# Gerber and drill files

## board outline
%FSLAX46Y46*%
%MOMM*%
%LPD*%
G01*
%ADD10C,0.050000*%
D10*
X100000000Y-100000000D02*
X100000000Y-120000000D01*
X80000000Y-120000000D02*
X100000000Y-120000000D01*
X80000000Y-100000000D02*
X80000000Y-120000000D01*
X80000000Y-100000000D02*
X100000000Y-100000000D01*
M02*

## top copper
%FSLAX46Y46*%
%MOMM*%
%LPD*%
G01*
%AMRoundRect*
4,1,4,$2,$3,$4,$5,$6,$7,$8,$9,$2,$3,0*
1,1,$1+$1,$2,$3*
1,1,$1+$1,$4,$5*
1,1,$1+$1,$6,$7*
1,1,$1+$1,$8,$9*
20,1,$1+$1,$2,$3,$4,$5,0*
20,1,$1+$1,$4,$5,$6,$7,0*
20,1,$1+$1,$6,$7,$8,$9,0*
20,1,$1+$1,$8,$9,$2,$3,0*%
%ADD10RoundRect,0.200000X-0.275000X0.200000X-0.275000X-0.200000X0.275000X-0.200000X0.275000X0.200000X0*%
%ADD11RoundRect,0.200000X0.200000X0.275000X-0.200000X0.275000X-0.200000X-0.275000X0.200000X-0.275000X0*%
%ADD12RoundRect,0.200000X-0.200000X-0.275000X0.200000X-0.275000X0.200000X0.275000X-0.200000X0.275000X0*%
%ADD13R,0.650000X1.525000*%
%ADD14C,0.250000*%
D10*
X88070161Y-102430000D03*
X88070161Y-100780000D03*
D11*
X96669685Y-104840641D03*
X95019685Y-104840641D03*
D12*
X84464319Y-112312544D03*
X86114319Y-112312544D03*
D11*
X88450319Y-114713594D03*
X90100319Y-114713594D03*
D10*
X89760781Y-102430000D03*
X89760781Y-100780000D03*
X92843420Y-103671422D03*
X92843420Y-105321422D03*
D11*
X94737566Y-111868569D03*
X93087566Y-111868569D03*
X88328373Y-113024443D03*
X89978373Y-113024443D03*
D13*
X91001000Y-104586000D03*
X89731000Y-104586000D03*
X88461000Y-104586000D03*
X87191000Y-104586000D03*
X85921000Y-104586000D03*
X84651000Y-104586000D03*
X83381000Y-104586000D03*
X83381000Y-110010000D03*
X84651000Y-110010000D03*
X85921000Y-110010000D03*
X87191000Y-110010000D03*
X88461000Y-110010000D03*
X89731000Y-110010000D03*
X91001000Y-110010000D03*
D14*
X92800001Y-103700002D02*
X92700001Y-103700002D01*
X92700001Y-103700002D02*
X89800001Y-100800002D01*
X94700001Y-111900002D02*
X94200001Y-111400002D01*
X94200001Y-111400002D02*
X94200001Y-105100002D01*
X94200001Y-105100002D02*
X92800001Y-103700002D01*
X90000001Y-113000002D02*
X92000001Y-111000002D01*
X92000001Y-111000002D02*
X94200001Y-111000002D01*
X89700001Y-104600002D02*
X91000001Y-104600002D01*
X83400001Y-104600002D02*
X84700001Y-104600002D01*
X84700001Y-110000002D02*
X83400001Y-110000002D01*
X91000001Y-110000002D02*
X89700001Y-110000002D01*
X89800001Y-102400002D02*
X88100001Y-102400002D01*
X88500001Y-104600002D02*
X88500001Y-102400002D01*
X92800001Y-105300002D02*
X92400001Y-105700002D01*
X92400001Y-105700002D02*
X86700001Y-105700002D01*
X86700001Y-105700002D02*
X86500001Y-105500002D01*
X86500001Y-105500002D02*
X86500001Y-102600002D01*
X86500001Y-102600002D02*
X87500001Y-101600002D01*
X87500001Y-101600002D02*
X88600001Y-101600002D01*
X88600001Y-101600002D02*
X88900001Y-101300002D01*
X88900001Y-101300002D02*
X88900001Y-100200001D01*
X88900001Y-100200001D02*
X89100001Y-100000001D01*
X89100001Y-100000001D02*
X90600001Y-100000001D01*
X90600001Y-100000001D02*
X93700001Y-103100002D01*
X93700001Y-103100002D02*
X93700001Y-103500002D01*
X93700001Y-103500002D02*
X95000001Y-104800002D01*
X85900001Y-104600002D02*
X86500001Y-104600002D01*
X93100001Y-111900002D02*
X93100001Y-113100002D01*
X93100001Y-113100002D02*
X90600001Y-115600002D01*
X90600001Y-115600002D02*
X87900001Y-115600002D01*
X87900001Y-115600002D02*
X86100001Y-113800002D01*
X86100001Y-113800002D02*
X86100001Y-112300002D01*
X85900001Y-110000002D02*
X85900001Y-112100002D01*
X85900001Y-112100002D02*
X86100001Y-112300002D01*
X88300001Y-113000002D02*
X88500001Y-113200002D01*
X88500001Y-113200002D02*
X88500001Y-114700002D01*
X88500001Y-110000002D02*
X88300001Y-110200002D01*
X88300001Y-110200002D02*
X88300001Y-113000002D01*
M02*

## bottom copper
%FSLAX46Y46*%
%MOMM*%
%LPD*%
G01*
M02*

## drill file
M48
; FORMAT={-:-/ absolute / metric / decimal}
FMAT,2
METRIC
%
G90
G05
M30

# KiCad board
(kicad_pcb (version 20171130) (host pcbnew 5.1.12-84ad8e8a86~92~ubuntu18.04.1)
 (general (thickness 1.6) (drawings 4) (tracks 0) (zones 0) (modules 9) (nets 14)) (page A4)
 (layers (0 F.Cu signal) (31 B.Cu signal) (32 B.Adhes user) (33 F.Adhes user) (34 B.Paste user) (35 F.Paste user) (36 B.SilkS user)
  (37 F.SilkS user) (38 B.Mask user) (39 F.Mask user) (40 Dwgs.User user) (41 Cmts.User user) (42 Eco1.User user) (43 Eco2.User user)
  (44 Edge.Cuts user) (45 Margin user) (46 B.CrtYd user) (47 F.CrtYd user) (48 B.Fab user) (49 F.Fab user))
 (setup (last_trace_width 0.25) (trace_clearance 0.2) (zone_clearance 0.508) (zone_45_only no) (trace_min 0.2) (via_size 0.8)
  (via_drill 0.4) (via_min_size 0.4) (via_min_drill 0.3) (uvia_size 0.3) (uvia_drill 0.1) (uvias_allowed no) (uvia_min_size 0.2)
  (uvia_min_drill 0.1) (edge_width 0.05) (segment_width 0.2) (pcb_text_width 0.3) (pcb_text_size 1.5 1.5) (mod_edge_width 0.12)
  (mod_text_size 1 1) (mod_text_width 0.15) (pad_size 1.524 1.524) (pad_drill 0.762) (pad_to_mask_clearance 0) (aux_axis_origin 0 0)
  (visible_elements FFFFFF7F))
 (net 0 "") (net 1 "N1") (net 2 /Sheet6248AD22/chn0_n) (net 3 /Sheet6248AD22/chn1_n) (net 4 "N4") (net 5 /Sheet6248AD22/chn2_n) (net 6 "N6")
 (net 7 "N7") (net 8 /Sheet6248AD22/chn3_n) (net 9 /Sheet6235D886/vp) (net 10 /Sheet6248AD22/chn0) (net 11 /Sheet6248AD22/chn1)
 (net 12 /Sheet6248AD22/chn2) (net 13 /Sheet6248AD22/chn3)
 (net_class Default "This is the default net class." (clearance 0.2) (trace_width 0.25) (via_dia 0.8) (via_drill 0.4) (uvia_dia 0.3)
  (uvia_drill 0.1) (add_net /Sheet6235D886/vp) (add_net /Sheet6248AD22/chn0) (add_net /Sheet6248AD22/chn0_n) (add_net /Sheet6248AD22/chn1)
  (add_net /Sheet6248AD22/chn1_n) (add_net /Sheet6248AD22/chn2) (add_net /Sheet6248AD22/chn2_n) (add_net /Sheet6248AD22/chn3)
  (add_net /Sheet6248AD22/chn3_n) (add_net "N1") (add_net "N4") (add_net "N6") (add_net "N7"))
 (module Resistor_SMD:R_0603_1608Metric (layer F.Cu) (at 88.070161 101.605000 270.000000)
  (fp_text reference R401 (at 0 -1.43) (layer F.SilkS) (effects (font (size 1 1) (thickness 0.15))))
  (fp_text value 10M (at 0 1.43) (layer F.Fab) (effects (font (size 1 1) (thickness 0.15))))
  (pad 2 smd roundrect (at 0.825 0 270.000000) (size 0.8 0.95) (layers F.Cu F.Mask F.Paste) (roundrect_rratio 0.25) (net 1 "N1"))
  (pad 1 smd roundrect (at -0.825 0 270.000000) (size 0.8 0.95) (layers F.Cu F.Mask F.Paste) (roundrect_rratio 0.25)
   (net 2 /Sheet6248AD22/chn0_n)))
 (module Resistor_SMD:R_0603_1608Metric (layer F.Cu) (at 95.844685 104.840641 180.000000)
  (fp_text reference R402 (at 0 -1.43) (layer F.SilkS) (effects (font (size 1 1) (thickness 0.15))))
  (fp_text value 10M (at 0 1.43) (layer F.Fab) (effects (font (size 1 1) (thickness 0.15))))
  (pad 1 smd roundrect (at -0.825 0 180.000000) (size 0.8 0.95) (layers F.Cu F.Mask F.Paste) (roundrect_rratio 0.25)
   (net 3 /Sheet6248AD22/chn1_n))
  (pad 2 smd roundrect (at 0.825 0 180.000000) (size 0.8 0.95) (layers F.Cu F.Mask F.Paste) (roundrect_rratio 0.25) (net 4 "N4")))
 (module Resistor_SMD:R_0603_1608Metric (layer F.Cu) (at 85.289319 112.312544)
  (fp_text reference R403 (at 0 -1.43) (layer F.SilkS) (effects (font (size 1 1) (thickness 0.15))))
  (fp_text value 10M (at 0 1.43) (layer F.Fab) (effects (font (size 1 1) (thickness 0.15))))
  (pad 1 smd roundrect (at -0.825 0) (size 0.8 0.95) (layers F.Cu F.Mask F.Paste) (roundrect_rratio 0.25) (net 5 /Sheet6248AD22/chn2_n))
  (pad 2 smd roundrect (at 0.825 0) (size 0.8 0.95) (layers F.Cu F.Mask F.Paste) (roundrect_rratio 0.25) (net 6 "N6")))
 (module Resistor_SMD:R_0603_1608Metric (layer F.Cu) (at 89.275319 114.713594 180.000000)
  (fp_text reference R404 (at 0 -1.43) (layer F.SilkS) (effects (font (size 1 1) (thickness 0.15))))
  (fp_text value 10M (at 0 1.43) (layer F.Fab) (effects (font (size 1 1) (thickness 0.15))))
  (pad 2 smd roundrect (at 0.825 0 180.000000) (size 0.8 0.95) (layers F.Cu F.Mask F.Paste) (roundrect_rratio 0.25) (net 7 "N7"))
  (pad 1 smd roundrect (at -0.825 0 180.000000) (size 0.8 0.95) (layers F.Cu F.Mask F.Paste) (roundrect_rratio 0.25)
   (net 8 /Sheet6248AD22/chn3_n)))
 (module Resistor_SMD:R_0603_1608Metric (layer F.Cu) (at 89.760781 101.605000 270.000000)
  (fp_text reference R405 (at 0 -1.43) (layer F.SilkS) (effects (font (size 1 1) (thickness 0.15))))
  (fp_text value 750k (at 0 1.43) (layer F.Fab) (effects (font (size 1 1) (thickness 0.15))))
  (pad 2 smd roundrect (at 0.825 0 270.000000) (size 0.8 0.95) (layers F.Cu F.Mask F.Paste) (roundrect_rratio 0.25) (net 1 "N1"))
  (pad 1 smd roundrect (at -0.825 0 270.000000) (size 0.8 0.95) (layers F.Cu F.Mask F.Paste) (roundrect_rratio 0.25)
   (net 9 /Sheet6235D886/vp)))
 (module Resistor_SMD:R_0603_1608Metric (layer F.Cu) (at 92.843420 104.496422 270.000000)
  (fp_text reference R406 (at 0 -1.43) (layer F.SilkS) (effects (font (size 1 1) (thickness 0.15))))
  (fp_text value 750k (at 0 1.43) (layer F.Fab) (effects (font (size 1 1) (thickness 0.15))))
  (pad 1 smd roundrect (at -0.825 0 270.000000) (size 0.8 0.95) (layers F.Cu F.Mask F.Paste) (roundrect_rratio 0.25)
   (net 9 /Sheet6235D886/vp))
  (pad 2 smd roundrect (at 0.825 0 270.000000) (size 0.8 0.95) (layers F.Cu F.Mask F.Paste) (roundrect_rratio 0.25) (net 4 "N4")))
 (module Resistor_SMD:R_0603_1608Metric (layer F.Cu) (at 93.912566 111.868569 180.000000)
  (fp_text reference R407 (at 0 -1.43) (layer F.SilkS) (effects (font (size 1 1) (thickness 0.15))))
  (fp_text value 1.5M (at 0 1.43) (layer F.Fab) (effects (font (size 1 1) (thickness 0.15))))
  (pad 1 smd roundrect (at -0.825 0 180.000000) (size 0.8 0.95) (layers F.Cu F.Mask F.Paste) (roundrect_rratio 0.25)
   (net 9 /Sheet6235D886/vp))
  (pad 2 smd roundrect (at 0.825 0 180.000000) (size 0.8 0.95) (layers F.Cu F.Mask F.Paste) (roundrect_rratio 0.25) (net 6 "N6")))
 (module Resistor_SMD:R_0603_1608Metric (layer F.Cu) (at 89.153373 113.024443 180.000000)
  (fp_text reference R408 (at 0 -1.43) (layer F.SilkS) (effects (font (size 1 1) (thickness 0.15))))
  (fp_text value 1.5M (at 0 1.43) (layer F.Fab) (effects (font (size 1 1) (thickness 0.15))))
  (pad 2 smd roundrect (at 0.825 0 180.000000) (size 0.8 0.95) (layers F.Cu F.Mask F.Paste) (roundrect_rratio 0.25) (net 7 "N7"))
  (pad 1 smd roundrect (at -0.825 0 180.000000) (size 0.8 0.95) (layers F.Cu F.Mask F.Paste) (roundrect_rratio 0.25)
   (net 9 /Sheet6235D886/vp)))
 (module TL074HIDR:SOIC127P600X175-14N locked (layer F.Cu) (at 87.191000 107.298000 270.000000)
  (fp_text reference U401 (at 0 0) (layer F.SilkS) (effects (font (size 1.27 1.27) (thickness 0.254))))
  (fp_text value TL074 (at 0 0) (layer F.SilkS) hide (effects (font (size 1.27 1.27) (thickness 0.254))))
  (pad 1 smd rect (at -2.712 -3.81) (size 0.65 1.525) (layers F.Cu F.Mask F.Paste) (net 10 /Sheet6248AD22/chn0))
  (pad 2 smd rect (at -2.712 -2.54) (size 0.65 1.525) (layers F.Cu F.Mask F.Paste) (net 10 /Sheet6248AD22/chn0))
  (pad 3 smd rect (at -2.712 -1.27) (size 0.65 1.525) (layers F.Cu F.Mask F.Paste) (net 1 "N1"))
  (pad 4 smd rect (at -2.712 0) (size 0.65 1.525) (layers F.Cu F.Mask F.Paste))
  (pad 5 smd rect (at -2.712 1.27) (size 0.65 1.525) (layers F.Cu F.Mask F.Paste) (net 4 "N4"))
  (pad 6 smd rect (at -2.712 2.54) (size 0.65 1.525) (layers F.Cu F.Mask F.Paste) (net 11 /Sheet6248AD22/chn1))
  (pad 7 smd rect (at -2.712 3.81) (size 0.65 1.525) (layers F.Cu F.Mask F.Paste) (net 11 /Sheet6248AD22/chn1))
  (pad 8 smd rect (at 2.712 3.81) (size 0.65 1.525) (layers F.Cu F.Mask F.Paste) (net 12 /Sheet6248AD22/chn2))
  (pad 9 smd rect (at 2.712 2.54) (size 0.65 1.525) (layers F.Cu F.Mask F.Paste) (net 12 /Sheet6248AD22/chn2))
  (pad 10 smd rect (at 2.712 1.27) (size 0.65 1.525) (layers F.Cu F.Mask F.Paste) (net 6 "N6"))
  (pad 11 smd rect (at 2.712 0) (size 0.65 1.525) (layers F.Cu F.Mask F.Paste))
  (pad 12 smd rect (at 2.712 -1.27) (size 0.65 1.525) (layers F.Cu F.Mask F.Paste) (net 7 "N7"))
  (pad 13 smd rect (at 2.712 -2.54) (size 0.65 1.525) (layers F.Cu F.Mask F.Paste) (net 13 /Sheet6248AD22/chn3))
  (pad 14 smd rect (at 2.712 -3.81) (size 0.65 1.525) (layers F.Cu F.Mask F.Paste) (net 13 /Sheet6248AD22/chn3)))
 (gr_line (start 100 100) (end 100 120) (layer Edge.Cuts) (width 0.05))
 (gr_line (start 80 120) (end 100 120) (layer Edge.Cuts) (width 0.05))
 (gr_line (start 80 100) (end 80 120) (layer Edge.Cuts) (width 0.05))
 (gr_line (start 80 100) (end 100 100) (layer Edge.Cuts) (width 0.05))
 (segment (start 92.800001 103.700002) (end 92.700001 103.700002) (width 0.250000) (layer F.Cu) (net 9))
 (segment (start 92.700001 103.700002) (end 89.800001 100.800002) (width 0.250000) (layer F.Cu) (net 9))
 (segment (start 94.700001 111.900002) (end 94.200001 111.400002) (width 0.250000) (layer F.Cu) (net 9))
 (segment (start 94.200001 111.400002) (end 94.200001 105.100002) (width 0.250000) (layer F.Cu) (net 9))
 (segment (start 94.200001 105.100002) (end 92.800001 103.700002) (width 0.250000) (layer F.Cu) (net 9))
 (segment (start 90.000001 113.000002) (end 92.000001 111.000002) (width 0.250000) (layer F.Cu) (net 9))
 (segment (start 92.000001 111.000002) (end 94.200001 111.000002) (width 0.250000) (layer F.Cu) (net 9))
 (segment (start 89.700001 104.600002) (end 91.000001 104.600002) (width 0.250000) (layer F.Cu) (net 10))
 (segment (start 83.400001 104.600002) (end 84.700001 104.600002) (width 0.250000) (layer F.Cu) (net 11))
 (segment (start 84.700001 110.000002) (end 83.400001 110.000002) (width 0.250000) (layer F.Cu) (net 12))
 (segment (start 91.000001 110.000002) (end 89.700001 110.000002) (width 0.250000) (layer F.Cu) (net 13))
 (segment (start 89.800001 102.400002) (end 88.100001 102.400002) (width 0.250000) (layer F.Cu) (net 1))
 (segment (start 88.500001 104.600002) (end 88.500001 102.400002) (width 0.250000) (layer F.Cu) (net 1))
 (segment (start 92.800001 105.300002) (end 92.400001 105.700002) (width 0.250000) (layer F.Cu) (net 4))
 (segment (start 92.400001 105.700002) (end 86.700001 105.700002) (width 0.250000) (layer F.Cu) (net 4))
 (segment (start 86.700001 105.700002) (end 86.500001 105.500002) (width 0.250000) (layer F.Cu) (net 4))
 (segment (start 86.500001 105.500002) (end 86.500001 102.600002) (width 0.250000) (layer F.Cu) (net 4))
 (segment (start 86.500001 102.600002) (end 87.500001 101.600002) (width 0.250000) (layer F.Cu) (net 4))
 (segment (start 87.500001 101.600002) (end 88.600001 101.600002) (width 0.250000) (layer F.Cu) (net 4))
 (segment (start 88.600001 101.600002) (end 88.900001 101.300002) (width 0.250000) (layer F.Cu) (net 4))
 (segment (start 88.900001 101.300002) (end 88.900001 100.200001) (width 0.250000) (layer F.Cu) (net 4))
 (segment (start 88.900001 100.200001) (end 89.100001 100.000001) (width 0.250000) (layer F.Cu) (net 4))
 (segment (start 89.100001 100.000001) (end 90.600001 100.000001) (width 0.250000) (layer F.Cu) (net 4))
 (segment (start 90.600001 100.000001) (end 93.700001 103.100002) (width 0.250000) (layer F.Cu) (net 4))
 (segment (start 93.700001 103.100002) (end 93.700001 103.500002) (width 0.250000) (layer F.Cu) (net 4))
 (segment (start 93.700001 103.500002) (end 95.000001 104.800002) (width 0.250000) (layer F.Cu) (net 4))
 (segment (start 85.900001 104.600002) (end 86.500001 104.600002) (width 0.250000) (layer F.Cu) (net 4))
 (segment (start 93.100001 111.900002) (end 93.100001 113.100002) (width 0.250000) (layer F.Cu) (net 6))
 (segment (start 93.100001 113.100002) (end 90.600001 115.600002) (width 0.250000) (layer F.Cu) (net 6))
 (segment (start 90.600001 115.600002) (end 87.900001 115.600002) (width 0.250000) (layer F.Cu) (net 6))
 (segment (start 87.900001 115.600002) (end 86.100001 113.800002) (width 0.250000) (layer F.Cu) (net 6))
 (segment (start 86.100001 113.800002) (end 86.100001 112.300002) (width 0.250000) (layer F.Cu) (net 6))
 (segment (start 85.900001 110.000002) (end 85.900001 112.100002) (width 0.250000) (layer F.Cu) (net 6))
 (segment (start 85.900001 112.100002) (end 86.100001 112.300002) (width 0.250000) (layer F.Cu) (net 6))
 (segment (start 88.300001 113.000002) (end 88.500001 113.200002) (width 0.250000) (layer F.Cu) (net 7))
 (segment (start 88.500001 113.200002) (end 88.500001 114.700002) (width 0.250000) (layer F.Cu) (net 7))
 (segment (start 88.500001 110.000002) (end 88.300001 110.200002) (width 0.250000) (layer F.Cu) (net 7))
 (segment (start 88.300001 110.200002) (end 88.300001 113.000002) (width 0.250000) (layer F.Cu) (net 7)))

